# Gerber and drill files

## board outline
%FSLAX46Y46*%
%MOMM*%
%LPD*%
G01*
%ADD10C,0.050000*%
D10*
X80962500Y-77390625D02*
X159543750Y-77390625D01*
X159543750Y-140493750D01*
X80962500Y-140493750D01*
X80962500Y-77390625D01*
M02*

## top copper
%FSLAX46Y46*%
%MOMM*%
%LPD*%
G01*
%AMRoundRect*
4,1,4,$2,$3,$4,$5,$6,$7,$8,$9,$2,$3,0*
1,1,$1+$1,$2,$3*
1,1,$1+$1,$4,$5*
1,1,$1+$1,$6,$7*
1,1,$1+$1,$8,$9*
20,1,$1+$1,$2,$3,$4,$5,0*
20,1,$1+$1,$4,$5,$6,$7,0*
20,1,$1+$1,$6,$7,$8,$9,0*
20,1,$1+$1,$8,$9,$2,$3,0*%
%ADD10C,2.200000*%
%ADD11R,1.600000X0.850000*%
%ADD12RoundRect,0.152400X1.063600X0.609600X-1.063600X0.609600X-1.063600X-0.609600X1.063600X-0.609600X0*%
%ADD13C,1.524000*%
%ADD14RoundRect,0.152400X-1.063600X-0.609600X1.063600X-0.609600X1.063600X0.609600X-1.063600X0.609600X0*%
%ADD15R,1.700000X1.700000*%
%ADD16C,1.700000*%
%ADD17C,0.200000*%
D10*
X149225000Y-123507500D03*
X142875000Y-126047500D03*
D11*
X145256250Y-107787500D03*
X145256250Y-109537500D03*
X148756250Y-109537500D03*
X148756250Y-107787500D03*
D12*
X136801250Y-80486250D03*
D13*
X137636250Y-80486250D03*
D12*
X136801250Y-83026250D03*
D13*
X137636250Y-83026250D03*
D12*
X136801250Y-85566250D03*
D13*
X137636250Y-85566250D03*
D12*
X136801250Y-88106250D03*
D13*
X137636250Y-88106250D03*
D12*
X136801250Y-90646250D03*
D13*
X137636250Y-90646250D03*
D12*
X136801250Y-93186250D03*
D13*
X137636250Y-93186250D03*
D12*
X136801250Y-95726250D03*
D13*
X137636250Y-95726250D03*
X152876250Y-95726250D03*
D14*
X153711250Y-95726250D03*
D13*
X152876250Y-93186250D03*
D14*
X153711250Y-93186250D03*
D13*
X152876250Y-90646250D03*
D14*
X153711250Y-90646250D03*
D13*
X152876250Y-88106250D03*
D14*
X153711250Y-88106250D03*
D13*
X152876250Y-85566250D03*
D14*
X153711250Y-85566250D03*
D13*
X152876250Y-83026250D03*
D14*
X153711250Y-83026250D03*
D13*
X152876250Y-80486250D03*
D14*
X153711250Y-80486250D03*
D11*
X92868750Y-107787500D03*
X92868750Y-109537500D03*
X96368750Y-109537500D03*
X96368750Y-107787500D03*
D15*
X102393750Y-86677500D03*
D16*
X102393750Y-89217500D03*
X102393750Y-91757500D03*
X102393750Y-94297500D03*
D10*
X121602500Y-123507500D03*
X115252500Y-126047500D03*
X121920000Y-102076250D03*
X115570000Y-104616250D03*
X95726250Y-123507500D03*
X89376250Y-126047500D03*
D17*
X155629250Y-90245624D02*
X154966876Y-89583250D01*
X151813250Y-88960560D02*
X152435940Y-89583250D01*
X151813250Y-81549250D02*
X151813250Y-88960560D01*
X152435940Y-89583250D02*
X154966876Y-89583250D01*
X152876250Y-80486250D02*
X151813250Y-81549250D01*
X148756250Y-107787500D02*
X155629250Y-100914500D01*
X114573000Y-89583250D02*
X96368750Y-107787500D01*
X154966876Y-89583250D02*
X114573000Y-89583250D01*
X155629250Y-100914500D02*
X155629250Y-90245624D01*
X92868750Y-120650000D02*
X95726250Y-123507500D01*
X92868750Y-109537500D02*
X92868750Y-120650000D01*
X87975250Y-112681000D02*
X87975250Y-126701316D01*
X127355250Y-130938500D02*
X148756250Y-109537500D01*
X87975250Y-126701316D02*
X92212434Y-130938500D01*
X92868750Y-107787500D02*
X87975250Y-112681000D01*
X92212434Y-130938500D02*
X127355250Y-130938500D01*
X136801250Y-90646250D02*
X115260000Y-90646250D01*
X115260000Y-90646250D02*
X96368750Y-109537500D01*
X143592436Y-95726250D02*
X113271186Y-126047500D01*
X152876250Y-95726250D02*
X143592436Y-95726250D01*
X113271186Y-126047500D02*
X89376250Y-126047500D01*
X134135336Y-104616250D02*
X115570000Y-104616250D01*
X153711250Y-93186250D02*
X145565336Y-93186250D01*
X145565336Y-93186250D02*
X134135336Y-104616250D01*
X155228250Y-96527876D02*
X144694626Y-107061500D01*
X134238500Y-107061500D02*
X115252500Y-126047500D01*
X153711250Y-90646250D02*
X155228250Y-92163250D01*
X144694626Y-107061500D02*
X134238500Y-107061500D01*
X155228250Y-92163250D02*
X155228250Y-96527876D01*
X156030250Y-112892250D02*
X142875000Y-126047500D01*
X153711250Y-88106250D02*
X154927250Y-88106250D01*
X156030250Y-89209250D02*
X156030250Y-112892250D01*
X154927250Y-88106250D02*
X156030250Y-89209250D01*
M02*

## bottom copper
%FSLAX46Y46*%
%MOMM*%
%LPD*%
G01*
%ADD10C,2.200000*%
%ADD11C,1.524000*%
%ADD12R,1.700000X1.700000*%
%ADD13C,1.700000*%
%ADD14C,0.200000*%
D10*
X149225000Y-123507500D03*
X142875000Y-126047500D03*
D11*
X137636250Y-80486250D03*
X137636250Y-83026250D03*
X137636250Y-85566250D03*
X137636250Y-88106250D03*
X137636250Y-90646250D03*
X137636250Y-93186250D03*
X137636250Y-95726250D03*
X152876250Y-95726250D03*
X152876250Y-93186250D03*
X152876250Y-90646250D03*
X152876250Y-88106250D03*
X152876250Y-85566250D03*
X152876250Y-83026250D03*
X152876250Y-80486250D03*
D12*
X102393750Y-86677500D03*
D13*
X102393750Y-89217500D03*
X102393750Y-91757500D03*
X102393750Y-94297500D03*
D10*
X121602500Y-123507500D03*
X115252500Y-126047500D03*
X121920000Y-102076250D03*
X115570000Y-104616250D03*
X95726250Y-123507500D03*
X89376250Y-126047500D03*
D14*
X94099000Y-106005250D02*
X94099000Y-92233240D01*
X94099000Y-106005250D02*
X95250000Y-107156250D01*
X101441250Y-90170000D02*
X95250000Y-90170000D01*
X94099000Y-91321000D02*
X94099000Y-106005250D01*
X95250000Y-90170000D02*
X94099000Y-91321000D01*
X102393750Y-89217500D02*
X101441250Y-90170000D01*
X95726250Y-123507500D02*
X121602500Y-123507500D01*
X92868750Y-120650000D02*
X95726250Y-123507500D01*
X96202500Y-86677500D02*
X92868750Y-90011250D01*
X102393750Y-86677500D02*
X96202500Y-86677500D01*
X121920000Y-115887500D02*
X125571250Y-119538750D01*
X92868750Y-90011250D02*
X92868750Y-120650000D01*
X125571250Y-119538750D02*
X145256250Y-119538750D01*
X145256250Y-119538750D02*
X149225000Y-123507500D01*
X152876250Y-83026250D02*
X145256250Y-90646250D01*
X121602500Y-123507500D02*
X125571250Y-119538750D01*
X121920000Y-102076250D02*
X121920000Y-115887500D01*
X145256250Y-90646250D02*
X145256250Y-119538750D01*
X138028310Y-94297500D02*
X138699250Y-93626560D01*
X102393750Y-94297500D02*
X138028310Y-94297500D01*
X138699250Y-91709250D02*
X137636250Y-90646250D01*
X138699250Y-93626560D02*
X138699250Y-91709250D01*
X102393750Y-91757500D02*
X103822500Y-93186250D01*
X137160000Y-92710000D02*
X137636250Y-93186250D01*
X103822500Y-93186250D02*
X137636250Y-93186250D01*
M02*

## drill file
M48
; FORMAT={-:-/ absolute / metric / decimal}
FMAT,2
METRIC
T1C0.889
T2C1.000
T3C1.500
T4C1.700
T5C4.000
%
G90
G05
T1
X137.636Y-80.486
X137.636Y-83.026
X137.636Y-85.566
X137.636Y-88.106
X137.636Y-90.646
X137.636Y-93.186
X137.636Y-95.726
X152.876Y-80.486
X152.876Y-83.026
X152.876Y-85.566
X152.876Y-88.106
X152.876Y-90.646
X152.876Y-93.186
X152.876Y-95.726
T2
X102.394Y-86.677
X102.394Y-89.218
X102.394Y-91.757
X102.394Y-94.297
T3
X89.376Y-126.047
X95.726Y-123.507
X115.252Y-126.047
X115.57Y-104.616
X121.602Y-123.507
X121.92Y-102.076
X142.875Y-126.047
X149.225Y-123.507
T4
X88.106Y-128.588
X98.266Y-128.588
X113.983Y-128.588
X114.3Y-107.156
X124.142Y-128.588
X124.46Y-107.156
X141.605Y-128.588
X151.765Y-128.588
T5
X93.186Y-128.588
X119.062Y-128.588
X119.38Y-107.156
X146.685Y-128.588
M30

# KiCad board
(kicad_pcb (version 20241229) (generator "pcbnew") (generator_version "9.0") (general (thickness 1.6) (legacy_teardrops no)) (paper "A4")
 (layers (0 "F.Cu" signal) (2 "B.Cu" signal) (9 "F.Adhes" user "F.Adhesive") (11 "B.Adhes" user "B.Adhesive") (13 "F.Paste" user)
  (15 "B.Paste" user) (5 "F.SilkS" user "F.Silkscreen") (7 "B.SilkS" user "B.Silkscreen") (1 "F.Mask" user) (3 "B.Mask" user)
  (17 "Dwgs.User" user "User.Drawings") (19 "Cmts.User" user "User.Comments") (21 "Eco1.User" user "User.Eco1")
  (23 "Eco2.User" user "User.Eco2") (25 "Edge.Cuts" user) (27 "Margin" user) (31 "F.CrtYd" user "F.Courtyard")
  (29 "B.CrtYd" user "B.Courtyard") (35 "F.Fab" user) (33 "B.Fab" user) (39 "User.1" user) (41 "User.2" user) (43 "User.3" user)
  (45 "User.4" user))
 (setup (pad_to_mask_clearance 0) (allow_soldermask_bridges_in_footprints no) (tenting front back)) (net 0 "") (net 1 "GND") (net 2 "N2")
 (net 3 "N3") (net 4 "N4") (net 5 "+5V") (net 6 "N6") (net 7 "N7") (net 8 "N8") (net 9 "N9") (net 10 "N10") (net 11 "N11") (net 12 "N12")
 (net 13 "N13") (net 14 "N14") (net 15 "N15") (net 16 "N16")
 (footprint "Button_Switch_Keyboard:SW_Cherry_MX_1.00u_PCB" (layer "F.Cu") (at 149.225 123.5075)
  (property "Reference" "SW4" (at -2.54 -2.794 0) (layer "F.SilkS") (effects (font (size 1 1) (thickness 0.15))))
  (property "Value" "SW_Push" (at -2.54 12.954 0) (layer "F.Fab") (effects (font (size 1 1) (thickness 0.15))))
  (pad "" np_thru_hole circle (at -7.62 5.08) (size 1.7 1.7) (drill 1.7) (layers "*.Cu" "*.Mask"))
  (pad "" np_thru_hole circle (at -2.54 5.08) (size 4 4) (drill 4) (layers "*.Cu" "*.Mask"))
  (pad "" np_thru_hole circle (at 2.54 5.08) (size 1.7 1.7) (drill 1.7) (layers "*.Cu" "*.Mask"))
  (pad "1" thru_hole circle (at 0 0) (size 2.2 2.2) (drill 1.5) (layers "*.Cu" "*.Mask") (remove_unused_layers no) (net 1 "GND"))
  (pad "2" thru_hole circle (at -6.35 2.54) (size 2.2 2.2) (drill 1.5) (layers "*.Cu" "*.Mask") (remove_unused_layers no) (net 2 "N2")))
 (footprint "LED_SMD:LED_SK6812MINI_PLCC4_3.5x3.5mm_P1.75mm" (layer "F.Cu") (at 147.00625 108.6625)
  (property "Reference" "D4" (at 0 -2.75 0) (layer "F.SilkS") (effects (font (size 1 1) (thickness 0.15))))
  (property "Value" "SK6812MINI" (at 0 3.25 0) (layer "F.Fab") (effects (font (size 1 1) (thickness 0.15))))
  (pad "1" smd rect (at -1.75 -0.875) (size 1.6 0.85) (layers "F.Cu" "F.Mask" "F.Paste") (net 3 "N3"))
  (pad "2" smd rect (at -1.75 0.875) (size 1.6 0.85) (layers "F.Cu" "F.Mask" "F.Paste") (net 1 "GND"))
  (pad "3" smd rect (at 1.75 0.875) (size 1.6 0.85) (layers "F.Cu" "F.Mask" "F.Paste") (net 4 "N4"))
  (pad "4" smd rect (at 1.75 -0.875) (size 1.6 0.85) (layers "F.Cu" "F.Mask" "F.Paste") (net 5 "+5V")))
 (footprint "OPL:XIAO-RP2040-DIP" (layer "F.Cu") (at 145.25625 88.10625)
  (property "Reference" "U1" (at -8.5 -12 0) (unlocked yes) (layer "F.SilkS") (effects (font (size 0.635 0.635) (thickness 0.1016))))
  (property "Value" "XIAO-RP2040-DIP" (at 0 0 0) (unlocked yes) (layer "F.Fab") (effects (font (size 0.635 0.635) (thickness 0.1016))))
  (pad "1" smd roundrect (at -8.455 -7.62 180) (size 2.432 1.524) (layers "F.Cu" "F.Mask") (roundrect_rratio 0.1) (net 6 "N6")
   (thermal_bridge_angle 45))
  (pad "1" thru_hole circle (at -7.62 -7.62 180) (size 1.524 1.524) (drill 0.889) (layers "*.Cu" "*.Mask") (remove_unused_layers no)
   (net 6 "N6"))
  (pad "2" smd roundrect (at -8.455 -5.08 180) (size 2.432 1.524) (layers "F.Cu" "F.Mask") (roundrect_rratio 0.1) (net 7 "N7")
   (thermal_bridge_angle 45))
  (pad "2" thru_hole circle (at -7.62 -5.08 180) (size 1.524 1.524) (drill 0.889) (layers "*.Cu" "*.Mask") (remove_unused_layers no)
   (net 7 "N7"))
  (pad "3" smd roundrect (at -8.455 -2.54 180) (size 2.432 1.524) (layers "F.Cu" "F.Mask") (roundrect_rratio 0.1) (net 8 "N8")
   (thermal_bridge_angle 45))
  (pad "3" thru_hole circle (at -7.62 -2.54 180) (size 1.524 1.524) (drill 0.889) (layers "*.Cu" "*.Mask") (remove_unused_layers no)
   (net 8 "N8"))
  (pad "4" smd roundrect (at -8.455 0 180) (size 2.432 1.524) (layers "F.Cu" "F.Mask") (roundrect_rratio 0.1) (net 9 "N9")
   (thermal_bridge_angle 45))
  (pad "4" thru_hole circle (at -7.62 0 180) (size 1.524 1.524) (drill 0.889) (layers "*.Cu" "*.Mask") (remove_unused_layers no)
   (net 9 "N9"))
  (pad "5" smd roundrect (at -8.455 2.54 180) (size 2.432 1.524) (layers "F.Cu" "F.Mask") (roundrect_rratio 0.1) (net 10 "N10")
   (thermal_bridge_angle 45))
  (pad "5" thru_hole circle (at -7.62 2.54 180) (size 1.524 1.524) (drill 0.889) (layers "*.Cu" "*.Mask") (remove_unused_layers no)
   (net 10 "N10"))
  (pad "6" smd roundrect (at -8.455 5.08 180) (size 2.432 1.524) (layers "F.Cu" "F.Mask") (roundrect_rratio 0.1) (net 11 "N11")
   (thermal_bridge_angle 45))
  (pad "6" thru_hole circle (at -7.62 5.08 180) (size 1.524 1.524) (drill 0.889) (layers "*.Cu" "*.Mask") (remove_unused_layers no)
   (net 11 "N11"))
  (pad "7" smd roundrect (at -8.455 7.62 180) (size 2.432 1.524) (layers "F.Cu" "F.Mask") (roundrect_rratio 0.1) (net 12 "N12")
   (thermal_bridge_angle 45))
  (pad "7" thru_hole circle (at -7.62 7.62 180) (size 1.524 1.524) (drill 0.889) (layers "*.Cu" "*.Mask") (remove_unused_layers no)
   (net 12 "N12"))
  (pad "8" thru_hole circle (at 7.62 7.62) (size 1.524 1.524) (drill 0.889) (layers "*.Cu" "*.Mask") (remove_unused_layers no)
   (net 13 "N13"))
  (pad "8" smd roundrect (at 8.455 7.62) (size 2.432 1.524) (layers "F.Cu" "F.Mask") (roundrect_rratio 0.1) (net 13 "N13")
   (thermal_bridge_angle 45))
  (pad "9" thru_hole circle (at 7.62 5.08) (size 1.524 1.524) (drill 0.889) (layers "*.Cu" "*.Mask") (remove_unused_layers no)
   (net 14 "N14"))
  (pad "9" smd roundrect (at 8.455 5.08) (size 2.432 1.524) (layers "F.Cu" "F.Mask") (roundrect_rratio 0.1) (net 14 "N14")
   (thermal_bridge_angle 45))
  (pad "10" thru_hole circle (at 7.62 2.54) (size 1.524 1.524) (drill 0.889) (layers "*.Cu" "*.Mask") (remove_unused_layers no)
   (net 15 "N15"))
  (pad "10" smd roundrect (at 8.455 2.54) (size 2.432 1.524) (layers "F.Cu" "F.Mask") (roundrect_rratio 0.1) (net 15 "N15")
   (thermal_bridge_angle 45))
  (pad "11" thru_hole circle (at 7.62 0) (size 1.524 1.524) (drill 0.889) (layers "*.Cu" "*.Mask") (remove_unused_layers no) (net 2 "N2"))
  (pad "11" smd roundrect (at 8.455 0) (size 2.432 1.524) (layers "F.Cu" "F.Mask") (roundrect_rratio 0.1) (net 2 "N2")
   (thermal_bridge_angle 45))
  (pad "12" thru_hole circle (at 7.62 -2.54) (size 1.524 1.524) (drill 0.889) (layers "*.Cu" "*.Mask") (remove_unused_layers no)
   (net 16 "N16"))
  (pad "12" smd roundrect (at 8.455 -2.54) (size 2.432 1.524) (layers "F.Cu" "F.Mask") (roundrect_rratio 0.1) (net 16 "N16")
   (thermal_bridge_angle 45))
  (pad "13" thru_hole circle (at 7.62 -5.08) (size 1.524 1.524) (drill 0.889) (layers "*.Cu" "*.Mask") (remove_unused_layers no)
   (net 1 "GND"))
  (pad "13" smd roundrect (at 8.455 -5.08) (size 2.432 1.524) (layers "F.Cu" "F.Mask") (roundrect_rratio 0.1) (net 1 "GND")
   (thermal_bridge_angle 45))
  (pad "14" thru_hole circle (at 7.62 -7.62) (size 1.524 1.524) (drill 0.889) (layers "*.Cu" "*.Mask") (remove_unused_layers no)
   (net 5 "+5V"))
  (pad "14" smd roundrect (at 8.455 -7.62) (size 2.432 1.524) (layers "F.Cu" "F.Mask") (roundrect_rratio 0.1) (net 5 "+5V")
   (thermal_bridge_angle 45)))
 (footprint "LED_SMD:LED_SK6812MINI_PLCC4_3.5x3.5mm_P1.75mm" (layer "F.Cu") (at 94.61875 108.6625)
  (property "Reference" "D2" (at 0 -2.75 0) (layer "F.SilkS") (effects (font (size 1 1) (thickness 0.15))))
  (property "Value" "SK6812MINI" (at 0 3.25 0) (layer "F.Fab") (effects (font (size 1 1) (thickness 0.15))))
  (pad "1" smd rect (at -1.75 -0.875) (size 1.6 0.85) (layers "F.Cu" "F.Mask" "F.Paste") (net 4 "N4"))
  (pad "2" smd rect (at -1.75 0.875) (size 1.6 0.85) (layers "F.Cu" "F.Mask" "F.Paste") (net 1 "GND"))
  (pad "3" smd rect (at 1.75 0.875) (size 1.6 0.85) (layers "F.Cu" "F.Mask" "F.Paste") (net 6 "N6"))
  (pad "4" smd rect (at 1.75 -0.875) (size 1.6 0.85) (layers "F.Cu" "F.Mask" "F.Paste") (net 5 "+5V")))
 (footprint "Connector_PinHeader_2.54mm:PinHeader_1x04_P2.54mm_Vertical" (layer "F.Cu") (at 102.39375 86.6775)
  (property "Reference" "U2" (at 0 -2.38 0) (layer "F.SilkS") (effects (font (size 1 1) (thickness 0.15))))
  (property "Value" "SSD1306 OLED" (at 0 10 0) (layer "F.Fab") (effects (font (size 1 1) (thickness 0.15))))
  (pad "1" thru_hole rect (at 0 0) (size 1.7 1.7) (drill 1) (layers "*.Cu" "*.Mask") (remove_unused_layers no) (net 1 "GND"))
  (pad "2" thru_hole circle (at 0 2.54) (size 1.7 1.7) (drill 1) (layers "*.Cu" "*.Mask") (remove_unused_layers no) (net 5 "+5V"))
  (pad "3" thru_hole circle (at 0 5.08) (size 1.7 1.7) (drill 1) (layers "*.Cu" "*.Mask") (remove_unused_layers no) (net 11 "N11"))
  (pad "4" thru_hole circle (at 0 7.62) (size 1.7 1.7) (drill 1) (layers "*.Cu" "*.Mask") (remove_unused_layers no) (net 10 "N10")))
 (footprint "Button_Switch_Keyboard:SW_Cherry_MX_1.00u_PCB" (layer "F.Cu") (at 121.6025 123.5075)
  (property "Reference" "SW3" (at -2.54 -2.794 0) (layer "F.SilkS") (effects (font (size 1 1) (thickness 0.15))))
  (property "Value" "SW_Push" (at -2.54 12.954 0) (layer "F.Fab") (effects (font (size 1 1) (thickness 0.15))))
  (pad "" np_thru_hole circle (at -7.62 5.08) (size 1.7 1.7) (drill 1.7) (layers "*.Cu" "*.Mask"))
  (pad "" np_thru_hole circle (at -2.54 5.08) (size 4 4) (drill 4) (layers "*.Cu" "*.Mask"))
  (pad "" np_thru_hole circle (at 2.54 5.08) (size 1.7 1.7) (drill 1.7) (layers "*.Cu" "*.Mask"))
  (pad "1" thru_hole circle (at 0 0) (size 2.2 2.2) (drill 1.5) (layers "*.Cu" "*.Mask") (remove_unused_layers no) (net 1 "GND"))
  (pad "2" thru_hole circle (at -6.35 2.54) (size 2.2 2.2) (drill 1.5) (layers "*.Cu" "*.Mask") (remove_unused_layers no) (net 15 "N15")))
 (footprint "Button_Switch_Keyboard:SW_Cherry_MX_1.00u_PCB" (layer "F.Cu") (at 121.92 102.07625)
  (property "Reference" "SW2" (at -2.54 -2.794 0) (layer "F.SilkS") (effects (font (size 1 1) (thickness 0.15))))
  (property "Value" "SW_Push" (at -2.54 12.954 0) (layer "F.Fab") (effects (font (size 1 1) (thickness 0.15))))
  (pad "" np_thru_hole circle (at -7.62 5.08) (size 1.7 1.7) (drill 1.7) (layers "*.Cu" "*.Mask"))
  (pad "" np_thru_hole circle (at -2.54 5.08) (size 4 4) (drill 4) (layers "*.Cu" "*.Mask"))
  (pad "" np_thru_hole circle (at 2.54 5.08) (size 1.7 1.7) (drill 1.7) (layers "*.Cu" "*.Mask"))
  (pad "1" thru_hole circle (at 0 0) (size 2.2 2.2) (drill 1.5) (layers "*.Cu" "*.Mask") (remove_unused_layers no) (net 1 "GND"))
  (pad "2" thru_hole circle (at -6.35 2.54) (size 2.2 2.2) (drill 1.5) (layers "*.Cu" "*.Mask") (remove_unused_layers no) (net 14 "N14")))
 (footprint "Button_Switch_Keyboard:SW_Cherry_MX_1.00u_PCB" (layer "F.Cu") (at 95.72625 123.5075)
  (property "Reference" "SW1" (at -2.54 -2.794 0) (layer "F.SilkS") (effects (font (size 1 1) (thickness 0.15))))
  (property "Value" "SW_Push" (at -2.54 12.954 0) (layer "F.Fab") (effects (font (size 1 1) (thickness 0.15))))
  (pad "" np_thru_hole circle (at -7.62 5.08) (size 1.7 1.7) (drill 1.7) (layers "*.Cu" "*.Mask"))
  (pad "" np_thru_hole circle (at -2.54 5.08) (size 4 4) (drill 4) (layers "*.Cu" "*.Mask"))
  (pad "" np_thru_hole circle (at 2.54 5.08) (size 1.7 1.7) (drill 1.7) (layers "*.Cu" "*.Mask"))
  (pad "1" thru_hole circle (at 0 0) (size 2.2 2.2) (drill 1.5) (layers "*.Cu" "*.Mask") (remove_unused_layers no) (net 1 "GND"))
  (pad "2" thru_hole circle (at -6.35 2.54) (size 2.2 2.2) (drill 1.5) (layers "*.Cu" "*.Mask") (remove_unused_layers no) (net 13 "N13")))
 (gr_rect (start 80.9625 77.390625) (end 159.54375 140.49375) (stroke (width 0.05) (type default)) (fill no) (layer "Edge.Cuts"))
 (segment (start 155.62925 90.245624) (end 154.966876 89.58325) (width 0.2) (layer "F.Cu") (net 5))
 (segment (start 151.81325 88.96056) (end 152.43594 89.58325) (width 0.2) (layer "F.Cu") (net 5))
 (segment (start 151.81325 81.54925) (end 151.81325 88.96056) (width 0.2) (layer "F.Cu") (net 5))
 (segment (start 152.43594 89.58325) (end 154.966876 89.58325) (width 0.2) (layer "F.Cu") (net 5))
 (segment (start 152.87625 80.48625) (end 151.81325 81.54925) (width 0.2) (layer "F.Cu") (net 5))
 (segment (start 148.75625 107.7875) (end 155.62925 100.9145) (width 0.2) (layer "F.Cu") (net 5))
 (segment (start 114.573 89.58325) (end 96.36875 107.7875) (width 0.2) (layer "F.Cu") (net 5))
 (segment (start 154.966876 89.58325) (end 114.573 89.58325) (width 0.2) (layer "F.Cu") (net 5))
 (segment (start 155.62925 100.9145) (end 155.62925 90.245624) (width 0.2) (layer "F.Cu") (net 5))
 (segment (start 94.099 106.00525) (end 94.099 92.23324) (width 0.2) (layer "B.Cu") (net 5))
 (segment (start 94.099 106.00525) (end 95.25 107.15625) (width 0.2) (layer "B.Cu") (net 5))
 (segment (start 101.44125 90.17) (end 95.25 90.17) (width 0.2) (layer "B.Cu") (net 5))
 (segment (start 94.099 91.321) (end 94.099 106.00525) (width 0.2) (layer "B.Cu") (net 5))
 (segment (start 95.25 90.17) (end 94.099 91.321) (width 0.2) (layer "B.Cu") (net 5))
 (segment (start 102.39375 89.2175) (end 101.44125 90.17) (width 0.2) (layer "B.Cu") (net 5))
 (segment (start 92.86875 120.65) (end 95.72625 123.5075) (width 0.2) (layer "F.Cu") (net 1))
 (segment (start 92.86875 109.5375) (end 92.86875 120.65) (width 0.2) (layer "F.Cu") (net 1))
 (segment (start 95.72625 123.5075) (end 121.6025 123.5075) (width 0.2) (layer "B.Cu") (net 1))
 (segment (start 92.86875 120.65) (end 95.72625 123.5075) (width 0.2) (layer "B.Cu") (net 1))
 (segment (start 96.2025 86.6775) (end 92.86875 90.01125) (width 0.2) (layer "B.Cu") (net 1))
 (segment (start 102.39375 86.6775) (end 96.2025 86.6775) (width 0.2) (layer "B.Cu") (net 1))
 (segment (start 121.92 115.8875) (end 125.57125 119.53875) (width 0.2) (layer "B.Cu") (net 1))
 (segment (start 92.86875 90.01125) (end 92.86875 120.65) (width 0.2) (layer "B.Cu") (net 1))
 (segment (start 125.57125 119.53875) (end 145.25625 119.53875) (width 0.2) (layer "B.Cu") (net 1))
 (segment (start 145.25625 119.53875) (end 149.225 123.5075) (width 0.2) (layer "B.Cu") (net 1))
 (segment (start 152.87625 83.02625) (end 145.25625 90.64625) (width 0.2) (layer "B.Cu") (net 1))
 (segment (start 121.6025 123.5075) (end 125.57125 119.53875) (width 0.2) (layer "B.Cu") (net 1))
 (segment (start 121.92 102.07625) (end 121.92 115.8875) (width 0.2) (layer "B.Cu") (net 1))
 (segment (start 145.25625 90.64625) (end 145.25625 119.53875) (width 0.2) (layer "B.Cu") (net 1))
 (segment (start 87.97525 112.681) (end 87.97525 126.701316) (width 0.2) (layer "F.Cu") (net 4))
 (segment (start 127.35525 130.9385) (end 148.75625 109.5375) (width 0.2) (layer "F.Cu") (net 4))
 (segment (start 87.97525 126.701316) (end 92.212434 130.9385) (width 0.2) (layer "F.Cu") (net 4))
 (segment (start 92.86875 107.7875) (end 87.97525 112.681) (width 0.2) (layer "F.Cu") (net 4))
 (segment (start 92.212434 130.9385) (end 127.35525 130.9385) (width 0.2) (layer "F.Cu") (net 4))
 (segment (start 136.80125 90.64625) (end 115.26 90.64625) (width 0.2) (layer "F.Cu") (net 6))
 (segment (start 115.26 90.64625) (end 96.36875 109.5375) (width 0.2) (layer "F.Cu") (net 6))
 (segment (start 143.592436 95.72625) (end 113.271186 126.0475) (width 0.2) (layer "F.Cu") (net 13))
 (segment (start 152.87625 95.72625) (end 143.592436 95.72625) (width 0.2) (layer "F.Cu") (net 13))
 (segment (start 113.271186 126.0475) (end 89.37625 126.0475) (width 0.2) (layer "F.Cu") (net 13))
 (segment (start 134.135336 104.61625) (end 115.57 104.61625) (width 0.2) (layer "F.Cu") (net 14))
 (segment (start 153.71125 93.18625) (end 145.565336 93.18625) (width 0.2) (layer "F.Cu") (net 14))
 (segment (start 145.565336 93.18625) (end 134.135336 104.61625) (width 0.2) (layer "F.Cu") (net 14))
 (segment (start 155.22825 96.527876) (end 144.694626 107.0615) (width 0.2) (layer "F.Cu") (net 15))
 (segment (start 134.2385 107.0615) (end 115.2525 126.0475) (width 0.2) (layer "F.Cu") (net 15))
 (segment (start 153.71125 90.64625) (end 155.22825 92.16325) (width 0.2) (layer "F.Cu") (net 15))
 (segment (start 144.694626 107.0615) (end 134.2385 107.0615) (width 0.2) (layer "F.Cu") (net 15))
 (segment (start 155.22825 92.16325) (end 155.22825 96.527876) (width 0.2) (layer "F.Cu") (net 15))
 (segment (start 156.03025 112.89225) (end 142.875 126.0475) (width 0.2) (layer "F.Cu") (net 2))
 (segment (start 153.71125 88.10625) (end 154.92725 88.10625) (width 0.2) (layer "F.Cu") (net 2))
 (segment (start 156.03025 89.20925) (end 156.03025 112.89225) (width 0.2) (layer "F.Cu") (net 2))
 (segment (start 154.92725 88.10625) (end 156.03025 89.20925) (width 0.2) (layer "F.Cu") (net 2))
 (segment (start 138.02831 94.2975) (end 138.69925 93.62656) (width 0.2) (layer "B.Cu") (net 10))
 (segment (start 102.39375 94.2975) (end 138.02831 94.2975) (width 0.2) (layer "B.Cu") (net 10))
 (segment (start 138.69925 91.70925) (end 137.63625 90.64625) (width 0.2) (layer "B.Cu") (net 10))
 (segment (start 138.69925 93.62656) (end 138.69925 91.70925) (width 0.2) (layer "B.Cu") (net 10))
 (segment (start 102.39375 91.7575) (end 103.8225 93.18625) (width 0.2) (layer "B.Cu") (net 11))
 (segment (start 137.16 92.71) (end 137.63625 93.18625) (width 0.2) (layer "B.Cu") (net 11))
 (segment (start 103.8225 93.18625) (end 137.63625 93.18625) (width 0.2) (layer "B.Cu") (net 11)))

